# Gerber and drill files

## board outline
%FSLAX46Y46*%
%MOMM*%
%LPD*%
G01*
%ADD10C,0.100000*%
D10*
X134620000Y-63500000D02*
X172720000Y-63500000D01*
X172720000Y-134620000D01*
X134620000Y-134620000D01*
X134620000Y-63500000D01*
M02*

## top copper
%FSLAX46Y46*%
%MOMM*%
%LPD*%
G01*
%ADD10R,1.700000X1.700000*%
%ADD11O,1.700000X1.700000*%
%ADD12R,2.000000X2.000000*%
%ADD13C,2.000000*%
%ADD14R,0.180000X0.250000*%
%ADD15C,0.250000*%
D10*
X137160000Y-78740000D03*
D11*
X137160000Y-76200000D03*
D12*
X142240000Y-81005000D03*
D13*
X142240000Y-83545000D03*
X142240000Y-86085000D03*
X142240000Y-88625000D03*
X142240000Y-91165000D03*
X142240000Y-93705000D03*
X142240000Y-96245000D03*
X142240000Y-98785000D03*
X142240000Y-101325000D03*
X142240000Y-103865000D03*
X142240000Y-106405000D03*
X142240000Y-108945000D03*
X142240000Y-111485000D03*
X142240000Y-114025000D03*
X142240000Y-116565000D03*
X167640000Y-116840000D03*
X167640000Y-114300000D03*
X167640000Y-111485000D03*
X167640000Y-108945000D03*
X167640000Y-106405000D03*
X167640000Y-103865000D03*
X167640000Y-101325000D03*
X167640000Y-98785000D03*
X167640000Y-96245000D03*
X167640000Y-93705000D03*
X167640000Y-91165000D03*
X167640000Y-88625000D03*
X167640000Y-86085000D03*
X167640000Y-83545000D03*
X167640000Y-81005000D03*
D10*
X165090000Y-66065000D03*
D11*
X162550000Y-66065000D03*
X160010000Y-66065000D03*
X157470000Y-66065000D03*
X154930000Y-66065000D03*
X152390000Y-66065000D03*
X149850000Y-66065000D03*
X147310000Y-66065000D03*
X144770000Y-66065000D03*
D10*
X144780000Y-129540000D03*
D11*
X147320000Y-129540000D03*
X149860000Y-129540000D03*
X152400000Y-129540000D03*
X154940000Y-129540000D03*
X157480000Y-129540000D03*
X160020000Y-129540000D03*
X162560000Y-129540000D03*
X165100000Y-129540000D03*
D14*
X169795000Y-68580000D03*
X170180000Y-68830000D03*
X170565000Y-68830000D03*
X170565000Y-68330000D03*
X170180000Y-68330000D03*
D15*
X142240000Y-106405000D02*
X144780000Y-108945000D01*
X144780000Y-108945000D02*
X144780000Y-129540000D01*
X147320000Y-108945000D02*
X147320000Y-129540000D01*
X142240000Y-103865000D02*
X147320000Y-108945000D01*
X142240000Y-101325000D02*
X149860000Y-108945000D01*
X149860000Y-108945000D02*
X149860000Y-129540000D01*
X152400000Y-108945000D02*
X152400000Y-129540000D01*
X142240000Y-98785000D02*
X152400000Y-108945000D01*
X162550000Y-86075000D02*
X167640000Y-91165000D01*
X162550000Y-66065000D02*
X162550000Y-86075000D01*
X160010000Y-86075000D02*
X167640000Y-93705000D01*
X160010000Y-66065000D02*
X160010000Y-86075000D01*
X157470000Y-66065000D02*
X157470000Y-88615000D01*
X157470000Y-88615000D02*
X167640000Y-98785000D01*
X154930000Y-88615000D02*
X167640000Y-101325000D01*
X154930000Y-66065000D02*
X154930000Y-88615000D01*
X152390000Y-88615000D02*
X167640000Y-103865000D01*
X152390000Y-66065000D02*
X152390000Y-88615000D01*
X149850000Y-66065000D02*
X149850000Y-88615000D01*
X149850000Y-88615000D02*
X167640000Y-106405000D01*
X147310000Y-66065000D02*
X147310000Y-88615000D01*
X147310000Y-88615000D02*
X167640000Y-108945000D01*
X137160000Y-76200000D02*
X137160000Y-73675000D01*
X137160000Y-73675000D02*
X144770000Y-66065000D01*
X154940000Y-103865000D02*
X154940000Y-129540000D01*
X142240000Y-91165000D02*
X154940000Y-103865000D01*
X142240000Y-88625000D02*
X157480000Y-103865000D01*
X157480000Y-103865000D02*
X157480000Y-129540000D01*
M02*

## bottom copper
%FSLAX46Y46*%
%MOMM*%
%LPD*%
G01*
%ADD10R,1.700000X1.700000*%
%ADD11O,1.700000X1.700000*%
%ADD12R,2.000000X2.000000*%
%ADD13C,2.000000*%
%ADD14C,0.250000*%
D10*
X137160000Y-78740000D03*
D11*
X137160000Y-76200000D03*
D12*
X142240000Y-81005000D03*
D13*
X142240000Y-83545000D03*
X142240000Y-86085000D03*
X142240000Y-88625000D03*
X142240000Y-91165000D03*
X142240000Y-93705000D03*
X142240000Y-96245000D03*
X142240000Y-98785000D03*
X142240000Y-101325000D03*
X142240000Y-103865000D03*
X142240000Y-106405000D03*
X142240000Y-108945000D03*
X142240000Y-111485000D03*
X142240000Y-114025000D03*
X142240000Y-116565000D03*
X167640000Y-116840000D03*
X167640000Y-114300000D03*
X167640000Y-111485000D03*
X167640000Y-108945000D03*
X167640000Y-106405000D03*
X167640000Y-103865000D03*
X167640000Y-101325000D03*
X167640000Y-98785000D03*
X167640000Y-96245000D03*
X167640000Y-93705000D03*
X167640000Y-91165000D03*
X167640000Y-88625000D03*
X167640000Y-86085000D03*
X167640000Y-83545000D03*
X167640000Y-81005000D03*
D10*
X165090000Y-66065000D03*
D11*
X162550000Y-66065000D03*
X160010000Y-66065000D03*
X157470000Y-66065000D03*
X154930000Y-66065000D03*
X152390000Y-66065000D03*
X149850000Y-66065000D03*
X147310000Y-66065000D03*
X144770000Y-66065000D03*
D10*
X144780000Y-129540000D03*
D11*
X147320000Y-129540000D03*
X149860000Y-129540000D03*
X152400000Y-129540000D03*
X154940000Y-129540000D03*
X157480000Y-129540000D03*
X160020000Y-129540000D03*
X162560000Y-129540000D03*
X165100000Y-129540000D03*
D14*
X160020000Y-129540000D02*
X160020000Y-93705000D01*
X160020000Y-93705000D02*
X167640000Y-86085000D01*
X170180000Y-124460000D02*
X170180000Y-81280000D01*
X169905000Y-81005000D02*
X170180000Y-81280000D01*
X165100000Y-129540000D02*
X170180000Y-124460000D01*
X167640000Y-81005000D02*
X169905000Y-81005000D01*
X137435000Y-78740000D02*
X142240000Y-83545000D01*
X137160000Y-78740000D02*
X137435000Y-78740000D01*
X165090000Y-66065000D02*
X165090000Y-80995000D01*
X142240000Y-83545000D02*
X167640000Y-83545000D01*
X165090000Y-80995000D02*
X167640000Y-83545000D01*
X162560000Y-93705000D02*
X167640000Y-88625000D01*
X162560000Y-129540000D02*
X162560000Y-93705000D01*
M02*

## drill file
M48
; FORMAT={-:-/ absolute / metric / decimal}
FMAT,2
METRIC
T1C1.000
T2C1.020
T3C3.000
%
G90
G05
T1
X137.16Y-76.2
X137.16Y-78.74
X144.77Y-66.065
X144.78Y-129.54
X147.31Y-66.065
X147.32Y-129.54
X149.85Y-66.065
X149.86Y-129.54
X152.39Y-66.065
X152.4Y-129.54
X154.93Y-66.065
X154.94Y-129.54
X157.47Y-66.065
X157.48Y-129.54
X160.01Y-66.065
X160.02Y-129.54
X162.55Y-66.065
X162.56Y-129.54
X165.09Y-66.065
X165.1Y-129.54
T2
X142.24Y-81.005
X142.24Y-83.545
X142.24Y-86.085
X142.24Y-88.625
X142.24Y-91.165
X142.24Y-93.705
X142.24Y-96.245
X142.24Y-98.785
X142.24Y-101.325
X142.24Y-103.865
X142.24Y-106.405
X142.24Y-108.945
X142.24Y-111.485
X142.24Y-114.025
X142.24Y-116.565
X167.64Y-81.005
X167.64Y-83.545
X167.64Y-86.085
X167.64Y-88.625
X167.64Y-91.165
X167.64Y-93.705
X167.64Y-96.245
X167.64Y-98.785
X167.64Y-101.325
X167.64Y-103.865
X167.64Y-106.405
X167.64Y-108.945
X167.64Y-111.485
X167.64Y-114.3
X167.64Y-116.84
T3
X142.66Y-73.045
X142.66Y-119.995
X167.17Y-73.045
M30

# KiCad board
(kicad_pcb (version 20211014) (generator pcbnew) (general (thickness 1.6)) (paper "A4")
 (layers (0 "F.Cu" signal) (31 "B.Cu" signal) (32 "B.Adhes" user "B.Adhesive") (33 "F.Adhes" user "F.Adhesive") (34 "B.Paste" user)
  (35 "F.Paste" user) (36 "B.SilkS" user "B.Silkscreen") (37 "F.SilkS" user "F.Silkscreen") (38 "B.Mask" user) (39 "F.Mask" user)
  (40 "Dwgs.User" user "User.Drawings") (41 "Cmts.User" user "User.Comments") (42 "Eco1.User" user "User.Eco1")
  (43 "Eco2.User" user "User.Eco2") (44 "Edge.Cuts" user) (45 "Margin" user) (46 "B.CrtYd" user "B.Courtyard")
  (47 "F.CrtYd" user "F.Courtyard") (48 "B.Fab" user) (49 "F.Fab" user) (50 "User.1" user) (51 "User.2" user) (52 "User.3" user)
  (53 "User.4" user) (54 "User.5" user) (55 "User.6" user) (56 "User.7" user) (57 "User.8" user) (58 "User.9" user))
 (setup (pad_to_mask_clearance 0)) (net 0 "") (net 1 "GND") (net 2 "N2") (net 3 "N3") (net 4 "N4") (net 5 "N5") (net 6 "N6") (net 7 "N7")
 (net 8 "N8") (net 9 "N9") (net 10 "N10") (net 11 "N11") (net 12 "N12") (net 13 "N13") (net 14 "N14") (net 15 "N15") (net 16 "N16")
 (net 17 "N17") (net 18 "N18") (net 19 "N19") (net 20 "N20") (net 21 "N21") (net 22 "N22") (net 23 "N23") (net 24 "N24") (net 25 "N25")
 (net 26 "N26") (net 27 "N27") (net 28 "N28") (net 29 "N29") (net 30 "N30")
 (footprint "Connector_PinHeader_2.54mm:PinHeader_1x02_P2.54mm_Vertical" (layer "F.Cu") (at 137.16 78.74 180)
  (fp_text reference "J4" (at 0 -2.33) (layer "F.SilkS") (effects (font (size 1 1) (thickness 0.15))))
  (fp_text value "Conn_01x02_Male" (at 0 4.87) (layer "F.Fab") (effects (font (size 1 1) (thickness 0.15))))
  (pad "1" thru_hole rect (at 0 0 180) (size 1.7 1.7) (drill 1) (layers *.Cu *.Mask) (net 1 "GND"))
  (pad "2" thru_hole oval (at 0 2.54 180) (size 1.7 1.7) (drill 1) (layers *.Cu *.Mask) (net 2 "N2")))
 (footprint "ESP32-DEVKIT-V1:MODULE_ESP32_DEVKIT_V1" (layer "F.Cu") (at 154.94 96.52)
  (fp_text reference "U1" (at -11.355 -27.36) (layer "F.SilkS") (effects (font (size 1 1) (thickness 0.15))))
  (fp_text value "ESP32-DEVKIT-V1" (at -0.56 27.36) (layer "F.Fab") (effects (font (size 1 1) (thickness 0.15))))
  (pad "" np_thru_hole circle (at -12.28 23.475) (size 3 3) (drill 3) (layers *.Cu *.Mask))
  (pad "" np_thru_hole circle (at 12.23 -23.475) (size 3 3) (drill 3) (layers *.Cu *.Mask))
  (pad "" np_thru_hole circle (at -12.28 -23.475) (size 3 3) (drill 3) (layers *.Cu *.Mask))
  (pad "1" thru_hole rect (at -12.7 -15.515) (size 2 2) (drill 1.02) (layers *.Cu *.Mask) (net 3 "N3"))
  (pad "2" thru_hole circle (at -12.7 -12.975) (size 2 2) (drill 1.02) (layers *.Cu *.Mask) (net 1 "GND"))
  (pad "3" thru_hole circle (at -12.7 -10.435) (size 2 2) (drill 1.02) (layers *.Cu *.Mask) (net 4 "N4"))
  (pad "4" thru_hole circle (at -12.7 -7.895) (size 2 2) (drill 1.02) (layers *.Cu *.Mask) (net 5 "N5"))
  (pad "5" thru_hole circle (at -12.7 -5.355) (size 2 2) (drill 1.02) (layers *.Cu *.Mask) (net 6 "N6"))
  (pad "6" thru_hole circle (at -12.7 -2.815) (size 2 2) (drill 1.02) (layers *.Cu *.Mask) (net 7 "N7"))
  (pad "7" thru_hole circle (at -12.7 -0.275) (size 2 2) (drill 1.02) (layers *.Cu *.Mask) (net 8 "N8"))
  (pad "8" thru_hole circle (at -12.7 2.265) (size 2 2) (drill 1.02) (layers *.Cu *.Mask) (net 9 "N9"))
  (pad "9" thru_hole circle (at -12.7 4.805) (size 2 2) (drill 1.02) (layers *.Cu *.Mask) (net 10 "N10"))
  (pad "10" thru_hole circle (at -12.7 7.345) (size 2 2) (drill 1.02) (layers *.Cu *.Mask) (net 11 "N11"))
  (pad "11" thru_hole circle (at -12.7 9.885) (size 2 2) (drill 1.02) (layers *.Cu *.Mask) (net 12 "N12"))
  (pad "12" thru_hole circle (at -12.7 12.425) (size 2 2) (drill 1.02) (layers *.Cu *.Mask) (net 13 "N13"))
  (pad "13" thru_hole circle (at -12.7 14.965) (size 2 2) (drill 1.02) (layers *.Cu *.Mask) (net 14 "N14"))
  (pad "14" thru_hole circle (at -12.7 17.505) (size 2 2) (drill 1.02) (layers *.Cu *.Mask) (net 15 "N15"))
  (pad "15" thru_hole circle (at -12.7 20.045) (size 2 2) (drill 1.02) (layers *.Cu *.Mask) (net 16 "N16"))
  (pad "16" thru_hole circle (at 12.7 20.32) (size 2 2) (drill 1.02) (layers *.Cu *.Mask) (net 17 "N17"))
  (pad "17" thru_hole circle (at 12.7 17.78) (size 2 2) (drill 1.02) (layers *.Cu *.Mask) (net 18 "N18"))
  (pad "18" thru_hole circle (at 12.7 14.965) (size 2 2) (drill 1.02) (layers *.Cu *.Mask) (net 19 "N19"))
  (pad "19" thru_hole circle (at 12.7 12.425) (size 2 2) (drill 1.02) (layers *.Cu *.Mask) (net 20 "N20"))
  (pad "20" thru_hole circle (at 12.7 9.885) (size 2 2) (drill 1.02) (layers *.Cu *.Mask) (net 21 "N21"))
  (pad "21" thru_hole circle (at 12.7 7.345) (size 2 2) (drill 1.02) (layers *.Cu *.Mask) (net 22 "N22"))
  (pad "22" thru_hole circle (at 12.7 4.805) (size 2 2) (drill 1.02) (layers *.Cu *.Mask) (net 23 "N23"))
  (pad "23" thru_hole circle (at 12.7 2.265) (size 2 2) (drill 1.02) (layers *.Cu *.Mask) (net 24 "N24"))
  (pad "24" thru_hole circle (at 12.7 -0.275) (size 2 2) (drill 1.02) (layers *.Cu *.Mask) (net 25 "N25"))
  (pad "25" thru_hole circle (at 12.7 -2.815) (size 2 2) (drill 1.02) (layers *.Cu *.Mask) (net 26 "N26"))
  (pad "26" thru_hole circle (at 12.7 -5.355) (size 2 2) (drill 1.02) (layers *.Cu *.Mask) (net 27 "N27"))
  (pad "27" thru_hole circle (at 12.7 -7.895) (size 2 2) (drill 1.02) (layers *.Cu *.Mask) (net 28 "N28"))
  (pad "28" thru_hole circle (at 12.7 -10.435) (size 2 2) (drill 1.02) (layers *.Cu *.Mask) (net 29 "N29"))
  (pad "29" thru_hole circle (at 12.7 -12.975) (size 2 2) (drill 1.02) (layers *.Cu *.Mask) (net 1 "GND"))
  (pad "30" thru_hole circle (at 12.7 -15.515) (size 2 2) (drill 1.02) (layers *.Cu *.Mask) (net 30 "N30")))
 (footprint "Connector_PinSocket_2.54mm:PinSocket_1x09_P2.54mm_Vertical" (layer "F.Cu") (at 165.09 66.065 -90)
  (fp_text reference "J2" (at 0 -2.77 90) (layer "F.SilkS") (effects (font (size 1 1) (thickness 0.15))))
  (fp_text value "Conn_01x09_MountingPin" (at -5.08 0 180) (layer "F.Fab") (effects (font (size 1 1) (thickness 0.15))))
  (pad "1" thru_hole rect (at 0 0 270) (size 1.7 1.7) (drill 1) (layers *.Cu *.Mask) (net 1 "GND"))
  (pad "2" thru_hole oval (at 0 2.54 270) (size 1.7 1.7) (drill 1) (layers *.Cu *.Mask) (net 27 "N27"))
  (pad "3" thru_hole oval (at 0 5.08 270) (size 1.7 1.7) (drill 1) (layers *.Cu *.Mask) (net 26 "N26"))
  (pad "4" thru_hole oval (at 0 7.62 270) (size 1.7 1.7) (drill 1) (layers *.Cu *.Mask) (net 24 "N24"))
  (pad "5" thru_hole oval (at 0 10.16 270) (size 1.7 1.7) (drill 1) (layers *.Cu *.Mask) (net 23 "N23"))
  (pad "6" thru_hole oval (at 0 12.7 270) (size 1.7 1.7) (drill 1) (layers *.Cu *.Mask) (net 22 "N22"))
  (pad "7" thru_hole oval (at 0 15.24 270) (size 1.7 1.7) (drill 1) (layers *.Cu *.Mask) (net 21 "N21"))
  (pad "8" thru_hole oval (at 0 17.78 270) (size 1.7 1.7) (drill 1) (layers *.Cu *.Mask) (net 20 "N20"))
  (pad "9" thru_hole oval (at 0 20.32 270) (size 1.7 1.7) (drill 1) (layers *.Cu *.Mask) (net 2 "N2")))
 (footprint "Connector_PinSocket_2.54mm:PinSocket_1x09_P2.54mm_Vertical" (layer "F.Cu") (at 144.78 129.54 90)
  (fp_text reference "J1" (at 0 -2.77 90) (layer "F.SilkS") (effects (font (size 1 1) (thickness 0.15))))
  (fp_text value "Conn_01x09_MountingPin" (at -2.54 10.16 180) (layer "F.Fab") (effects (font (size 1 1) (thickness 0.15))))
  (pad "1" thru_hole rect (at 0 0 90) (size 1.7 1.7) (drill 1) (layers *.Cu *.Mask) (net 12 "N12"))
  (pad "2" thru_hole oval (at 0 2.54 90) (size 1.7 1.7) (drill 1) (layers *.Cu *.Mask) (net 11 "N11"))
  (pad "3" thru_hole oval (at 0 5.08 90) (size 1.7 1.7) (drill 1) (layers *.Cu *.Mask) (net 10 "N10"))
  (pad "4" thru_hole oval (at 0 7.62 90) (size 1.7 1.7) (drill 1) (layers *.Cu *.Mask) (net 9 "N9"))
  (pad "5" thru_hole oval (at 0 10.16 90) (size 1.7 1.7) (drill 1) (layers *.Cu *.Mask) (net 6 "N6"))
  (pad "6" thru_hole oval (at 0 12.7 90) (size 1.7 1.7) (drill 1) (layers *.Cu *.Mask) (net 5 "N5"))
  (pad "7" thru_hole oval (at 0 15.24 90) (size 1.7 1.7) (drill 1) (layers *.Cu *.Mask) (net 29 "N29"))
  (pad "8" thru_hole oval (at 0 17.78 90) (size 1.7 1.7) (drill 1) (layers *.Cu *.Mask) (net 28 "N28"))
  (pad "9" thru_hole oval (at 0 20.32 90) (size 1.7 1.7) (drill 1) (layers *.Cu *.Mask) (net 30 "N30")))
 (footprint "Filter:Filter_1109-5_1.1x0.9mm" (layer "F.Cu") (at 170.18 68.58)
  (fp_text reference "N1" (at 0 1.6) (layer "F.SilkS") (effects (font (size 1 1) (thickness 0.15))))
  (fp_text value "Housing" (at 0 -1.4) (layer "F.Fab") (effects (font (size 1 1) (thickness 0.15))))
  (pad "1" smd rect (at -0.385 0 90) (size 0.25 0.18) (layers "F.Cu" "F.Paste" "F.Mask"))
  (pad "2" smd rect (at 0 0.25 90) (size 0.25 0.18) (layers "F.Cu" "F.Paste" "F.Mask"))
  (pad "3" smd rect (at 0.385 0.25 90) (size 0.25 0.18) (layers "F.Cu" "F.Paste" "F.Mask"))
  (pad "4" smd rect (at 0.385 -0.25 90) (size 0.25 0.18) (layers "F.Cu" "F.Paste" "F.Mask"))
  (pad "5" smd rect (at 0 -0.25 90) (size 0.25 0.18) (layers "F.Cu" "F.Paste" "F.Mask")))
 (gr_rect (start 172.72 134.62) (end 134.62 63.5) (layer "Edge.Cuts") (width 0.1) (fill none))
 (segment (start 142.24 106.405) (end 144.78 108.945) (width 0.25) (layer "F.Cu") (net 12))
 (segment (start 144.78 108.945) (end 144.78 129.54) (width 0.25) (layer "F.Cu") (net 12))
 (segment (start 147.32 108.945) (end 147.32 129.54) (width 0.25) (layer "F.Cu") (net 11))
 (segment (start 142.24 103.865) (end 147.32 108.945) (width 0.25) (layer "F.Cu") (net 11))
 (segment (start 142.24 101.325) (end 149.86 108.945) (width 0.25) (layer "F.Cu") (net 10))
 (segment (start 149.86 108.945) (end 149.86 129.54) (width 0.25) (layer "F.Cu") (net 10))
 (segment (start 152.4 108.945) (end 152.4 129.54) (width 0.25) (layer "F.Cu") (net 9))
 (segment (start 142.24 98.785) (end 152.4 108.945) (width 0.25) (layer "F.Cu") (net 9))
 (segment (start 160.02 129.54) (end 160.02 93.705) (width 0.25) (layer "B.Cu") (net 29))
 (segment (start 160.02 93.705) (end 167.64 86.085) (width 0.25) (layer "B.Cu") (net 29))
 (segment (start 170.18 124.46) (end 170.18 81.28) (width 0.25) (layer "B.Cu") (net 30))
 (segment (start 169.905 81.005) (end 170.18 81.28) (width 0.25) (layer "B.Cu") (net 30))
 (segment (start 165.1 129.54) (end 170.18 124.46) (width 0.25) (layer "B.Cu") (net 30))
 (segment (start 167.64 81.005) (end 169.905 81.005) (width 0.25) (layer "B.Cu") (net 30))
 (segment (start 137.435 78.74) (end 142.24 83.545) (width 0.25) (layer "B.Cu") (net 1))
 (segment (start 137.16 78.74) (end 137.435 78.74) (width 0.25) (layer "B.Cu") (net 1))
 (segment (start 165.09 66.065) (end 165.09 80.995) (width 0.25) (layer "B.Cu") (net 1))
 (segment (start 142.24 83.545) (end 167.64 83.545) (width 0.25) (layer "B.Cu") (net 1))
 (segment (start 165.09 80.995) (end 167.64 83.545) (width 0.25) (layer "B.Cu") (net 1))
 (segment (start 162.55 86.075) (end 167.64 91.165) (width 0.25) (layer "F.Cu") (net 27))
 (segment (start 162.55 66.065) (end 162.55 86.075) (width 0.25) (layer "F.Cu") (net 27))
 (segment (start 160.01 86.075) (end 167.64 93.705) (width 0.25) (layer "F.Cu") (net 26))
 (segment (start 160.01 66.065) (end 160.01 86.075) (width 0.25) (layer "F.Cu") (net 26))
 (segment (start 157.47 66.065) (end 157.47 88.615) (width 0.25) (layer "F.Cu") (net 24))
 (segment (start 157.47 88.615) (end 167.64 98.785) (width 0.25) (layer "F.Cu") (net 24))
 (segment (start 154.93 88.615) (end 167.64 101.325) (width 0.25) (layer "F.Cu") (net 23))
 (segment (start 154.93 66.065) (end 154.93 88.615) (width 0.25) (layer "F.Cu") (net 23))
 (segment (start 152.39 88.615) (end 167.64 103.865) (width 0.25) (layer "F.Cu") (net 22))
 (segment (start 152.39 66.065) (end 152.39 88.615) (width 0.25) (layer "F.Cu") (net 22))
 (segment (start 149.85 66.065) (end 149.85 88.615) (width 0.25) (layer "F.Cu") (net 21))
 (segment (start 149.85 88.615) (end 167.64 106.405) (width 0.25) (layer "F.Cu") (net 21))
 (segment (start 147.31 66.065) (end 147.31 88.615) (width 0.25) (layer "F.Cu") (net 20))
 (segment (start 147.31 88.615) (end 167.64 108.945) (width 0.25) (layer "F.Cu") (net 20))
 (segment (start 137.16 76.2) (end 137.16 73.675) (width 0.25) (layer "F.Cu") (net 2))
 (segment (start 137.16 73.675) (end 144.77 66.065) (width 0.25) (layer "F.Cu") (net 2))
 (segment (start 154.94 103.865) (end 154.94 129.54) (width 0.25) (layer "F.Cu") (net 6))
 (segment (start 142.24 91.165) (end 154.94 103.865) (width 0.25) (layer "F.Cu") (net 6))
 (segment (start 142.24 88.625) (end 157.48 103.865) (width 0.25) (layer "F.Cu") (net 5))
 (segment (start 157.48 103.865) (end 157.48 129.54) (width 0.25) (layer "F.Cu") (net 5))
 (segment (start 162.56 93.705) (end 167.64 88.625) (width 0.25) (layer "B.Cu") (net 28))
 (segment (start 162.56 129.54) (end 162.56 93.705) (width 0.25) (layer "B.Cu") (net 28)))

